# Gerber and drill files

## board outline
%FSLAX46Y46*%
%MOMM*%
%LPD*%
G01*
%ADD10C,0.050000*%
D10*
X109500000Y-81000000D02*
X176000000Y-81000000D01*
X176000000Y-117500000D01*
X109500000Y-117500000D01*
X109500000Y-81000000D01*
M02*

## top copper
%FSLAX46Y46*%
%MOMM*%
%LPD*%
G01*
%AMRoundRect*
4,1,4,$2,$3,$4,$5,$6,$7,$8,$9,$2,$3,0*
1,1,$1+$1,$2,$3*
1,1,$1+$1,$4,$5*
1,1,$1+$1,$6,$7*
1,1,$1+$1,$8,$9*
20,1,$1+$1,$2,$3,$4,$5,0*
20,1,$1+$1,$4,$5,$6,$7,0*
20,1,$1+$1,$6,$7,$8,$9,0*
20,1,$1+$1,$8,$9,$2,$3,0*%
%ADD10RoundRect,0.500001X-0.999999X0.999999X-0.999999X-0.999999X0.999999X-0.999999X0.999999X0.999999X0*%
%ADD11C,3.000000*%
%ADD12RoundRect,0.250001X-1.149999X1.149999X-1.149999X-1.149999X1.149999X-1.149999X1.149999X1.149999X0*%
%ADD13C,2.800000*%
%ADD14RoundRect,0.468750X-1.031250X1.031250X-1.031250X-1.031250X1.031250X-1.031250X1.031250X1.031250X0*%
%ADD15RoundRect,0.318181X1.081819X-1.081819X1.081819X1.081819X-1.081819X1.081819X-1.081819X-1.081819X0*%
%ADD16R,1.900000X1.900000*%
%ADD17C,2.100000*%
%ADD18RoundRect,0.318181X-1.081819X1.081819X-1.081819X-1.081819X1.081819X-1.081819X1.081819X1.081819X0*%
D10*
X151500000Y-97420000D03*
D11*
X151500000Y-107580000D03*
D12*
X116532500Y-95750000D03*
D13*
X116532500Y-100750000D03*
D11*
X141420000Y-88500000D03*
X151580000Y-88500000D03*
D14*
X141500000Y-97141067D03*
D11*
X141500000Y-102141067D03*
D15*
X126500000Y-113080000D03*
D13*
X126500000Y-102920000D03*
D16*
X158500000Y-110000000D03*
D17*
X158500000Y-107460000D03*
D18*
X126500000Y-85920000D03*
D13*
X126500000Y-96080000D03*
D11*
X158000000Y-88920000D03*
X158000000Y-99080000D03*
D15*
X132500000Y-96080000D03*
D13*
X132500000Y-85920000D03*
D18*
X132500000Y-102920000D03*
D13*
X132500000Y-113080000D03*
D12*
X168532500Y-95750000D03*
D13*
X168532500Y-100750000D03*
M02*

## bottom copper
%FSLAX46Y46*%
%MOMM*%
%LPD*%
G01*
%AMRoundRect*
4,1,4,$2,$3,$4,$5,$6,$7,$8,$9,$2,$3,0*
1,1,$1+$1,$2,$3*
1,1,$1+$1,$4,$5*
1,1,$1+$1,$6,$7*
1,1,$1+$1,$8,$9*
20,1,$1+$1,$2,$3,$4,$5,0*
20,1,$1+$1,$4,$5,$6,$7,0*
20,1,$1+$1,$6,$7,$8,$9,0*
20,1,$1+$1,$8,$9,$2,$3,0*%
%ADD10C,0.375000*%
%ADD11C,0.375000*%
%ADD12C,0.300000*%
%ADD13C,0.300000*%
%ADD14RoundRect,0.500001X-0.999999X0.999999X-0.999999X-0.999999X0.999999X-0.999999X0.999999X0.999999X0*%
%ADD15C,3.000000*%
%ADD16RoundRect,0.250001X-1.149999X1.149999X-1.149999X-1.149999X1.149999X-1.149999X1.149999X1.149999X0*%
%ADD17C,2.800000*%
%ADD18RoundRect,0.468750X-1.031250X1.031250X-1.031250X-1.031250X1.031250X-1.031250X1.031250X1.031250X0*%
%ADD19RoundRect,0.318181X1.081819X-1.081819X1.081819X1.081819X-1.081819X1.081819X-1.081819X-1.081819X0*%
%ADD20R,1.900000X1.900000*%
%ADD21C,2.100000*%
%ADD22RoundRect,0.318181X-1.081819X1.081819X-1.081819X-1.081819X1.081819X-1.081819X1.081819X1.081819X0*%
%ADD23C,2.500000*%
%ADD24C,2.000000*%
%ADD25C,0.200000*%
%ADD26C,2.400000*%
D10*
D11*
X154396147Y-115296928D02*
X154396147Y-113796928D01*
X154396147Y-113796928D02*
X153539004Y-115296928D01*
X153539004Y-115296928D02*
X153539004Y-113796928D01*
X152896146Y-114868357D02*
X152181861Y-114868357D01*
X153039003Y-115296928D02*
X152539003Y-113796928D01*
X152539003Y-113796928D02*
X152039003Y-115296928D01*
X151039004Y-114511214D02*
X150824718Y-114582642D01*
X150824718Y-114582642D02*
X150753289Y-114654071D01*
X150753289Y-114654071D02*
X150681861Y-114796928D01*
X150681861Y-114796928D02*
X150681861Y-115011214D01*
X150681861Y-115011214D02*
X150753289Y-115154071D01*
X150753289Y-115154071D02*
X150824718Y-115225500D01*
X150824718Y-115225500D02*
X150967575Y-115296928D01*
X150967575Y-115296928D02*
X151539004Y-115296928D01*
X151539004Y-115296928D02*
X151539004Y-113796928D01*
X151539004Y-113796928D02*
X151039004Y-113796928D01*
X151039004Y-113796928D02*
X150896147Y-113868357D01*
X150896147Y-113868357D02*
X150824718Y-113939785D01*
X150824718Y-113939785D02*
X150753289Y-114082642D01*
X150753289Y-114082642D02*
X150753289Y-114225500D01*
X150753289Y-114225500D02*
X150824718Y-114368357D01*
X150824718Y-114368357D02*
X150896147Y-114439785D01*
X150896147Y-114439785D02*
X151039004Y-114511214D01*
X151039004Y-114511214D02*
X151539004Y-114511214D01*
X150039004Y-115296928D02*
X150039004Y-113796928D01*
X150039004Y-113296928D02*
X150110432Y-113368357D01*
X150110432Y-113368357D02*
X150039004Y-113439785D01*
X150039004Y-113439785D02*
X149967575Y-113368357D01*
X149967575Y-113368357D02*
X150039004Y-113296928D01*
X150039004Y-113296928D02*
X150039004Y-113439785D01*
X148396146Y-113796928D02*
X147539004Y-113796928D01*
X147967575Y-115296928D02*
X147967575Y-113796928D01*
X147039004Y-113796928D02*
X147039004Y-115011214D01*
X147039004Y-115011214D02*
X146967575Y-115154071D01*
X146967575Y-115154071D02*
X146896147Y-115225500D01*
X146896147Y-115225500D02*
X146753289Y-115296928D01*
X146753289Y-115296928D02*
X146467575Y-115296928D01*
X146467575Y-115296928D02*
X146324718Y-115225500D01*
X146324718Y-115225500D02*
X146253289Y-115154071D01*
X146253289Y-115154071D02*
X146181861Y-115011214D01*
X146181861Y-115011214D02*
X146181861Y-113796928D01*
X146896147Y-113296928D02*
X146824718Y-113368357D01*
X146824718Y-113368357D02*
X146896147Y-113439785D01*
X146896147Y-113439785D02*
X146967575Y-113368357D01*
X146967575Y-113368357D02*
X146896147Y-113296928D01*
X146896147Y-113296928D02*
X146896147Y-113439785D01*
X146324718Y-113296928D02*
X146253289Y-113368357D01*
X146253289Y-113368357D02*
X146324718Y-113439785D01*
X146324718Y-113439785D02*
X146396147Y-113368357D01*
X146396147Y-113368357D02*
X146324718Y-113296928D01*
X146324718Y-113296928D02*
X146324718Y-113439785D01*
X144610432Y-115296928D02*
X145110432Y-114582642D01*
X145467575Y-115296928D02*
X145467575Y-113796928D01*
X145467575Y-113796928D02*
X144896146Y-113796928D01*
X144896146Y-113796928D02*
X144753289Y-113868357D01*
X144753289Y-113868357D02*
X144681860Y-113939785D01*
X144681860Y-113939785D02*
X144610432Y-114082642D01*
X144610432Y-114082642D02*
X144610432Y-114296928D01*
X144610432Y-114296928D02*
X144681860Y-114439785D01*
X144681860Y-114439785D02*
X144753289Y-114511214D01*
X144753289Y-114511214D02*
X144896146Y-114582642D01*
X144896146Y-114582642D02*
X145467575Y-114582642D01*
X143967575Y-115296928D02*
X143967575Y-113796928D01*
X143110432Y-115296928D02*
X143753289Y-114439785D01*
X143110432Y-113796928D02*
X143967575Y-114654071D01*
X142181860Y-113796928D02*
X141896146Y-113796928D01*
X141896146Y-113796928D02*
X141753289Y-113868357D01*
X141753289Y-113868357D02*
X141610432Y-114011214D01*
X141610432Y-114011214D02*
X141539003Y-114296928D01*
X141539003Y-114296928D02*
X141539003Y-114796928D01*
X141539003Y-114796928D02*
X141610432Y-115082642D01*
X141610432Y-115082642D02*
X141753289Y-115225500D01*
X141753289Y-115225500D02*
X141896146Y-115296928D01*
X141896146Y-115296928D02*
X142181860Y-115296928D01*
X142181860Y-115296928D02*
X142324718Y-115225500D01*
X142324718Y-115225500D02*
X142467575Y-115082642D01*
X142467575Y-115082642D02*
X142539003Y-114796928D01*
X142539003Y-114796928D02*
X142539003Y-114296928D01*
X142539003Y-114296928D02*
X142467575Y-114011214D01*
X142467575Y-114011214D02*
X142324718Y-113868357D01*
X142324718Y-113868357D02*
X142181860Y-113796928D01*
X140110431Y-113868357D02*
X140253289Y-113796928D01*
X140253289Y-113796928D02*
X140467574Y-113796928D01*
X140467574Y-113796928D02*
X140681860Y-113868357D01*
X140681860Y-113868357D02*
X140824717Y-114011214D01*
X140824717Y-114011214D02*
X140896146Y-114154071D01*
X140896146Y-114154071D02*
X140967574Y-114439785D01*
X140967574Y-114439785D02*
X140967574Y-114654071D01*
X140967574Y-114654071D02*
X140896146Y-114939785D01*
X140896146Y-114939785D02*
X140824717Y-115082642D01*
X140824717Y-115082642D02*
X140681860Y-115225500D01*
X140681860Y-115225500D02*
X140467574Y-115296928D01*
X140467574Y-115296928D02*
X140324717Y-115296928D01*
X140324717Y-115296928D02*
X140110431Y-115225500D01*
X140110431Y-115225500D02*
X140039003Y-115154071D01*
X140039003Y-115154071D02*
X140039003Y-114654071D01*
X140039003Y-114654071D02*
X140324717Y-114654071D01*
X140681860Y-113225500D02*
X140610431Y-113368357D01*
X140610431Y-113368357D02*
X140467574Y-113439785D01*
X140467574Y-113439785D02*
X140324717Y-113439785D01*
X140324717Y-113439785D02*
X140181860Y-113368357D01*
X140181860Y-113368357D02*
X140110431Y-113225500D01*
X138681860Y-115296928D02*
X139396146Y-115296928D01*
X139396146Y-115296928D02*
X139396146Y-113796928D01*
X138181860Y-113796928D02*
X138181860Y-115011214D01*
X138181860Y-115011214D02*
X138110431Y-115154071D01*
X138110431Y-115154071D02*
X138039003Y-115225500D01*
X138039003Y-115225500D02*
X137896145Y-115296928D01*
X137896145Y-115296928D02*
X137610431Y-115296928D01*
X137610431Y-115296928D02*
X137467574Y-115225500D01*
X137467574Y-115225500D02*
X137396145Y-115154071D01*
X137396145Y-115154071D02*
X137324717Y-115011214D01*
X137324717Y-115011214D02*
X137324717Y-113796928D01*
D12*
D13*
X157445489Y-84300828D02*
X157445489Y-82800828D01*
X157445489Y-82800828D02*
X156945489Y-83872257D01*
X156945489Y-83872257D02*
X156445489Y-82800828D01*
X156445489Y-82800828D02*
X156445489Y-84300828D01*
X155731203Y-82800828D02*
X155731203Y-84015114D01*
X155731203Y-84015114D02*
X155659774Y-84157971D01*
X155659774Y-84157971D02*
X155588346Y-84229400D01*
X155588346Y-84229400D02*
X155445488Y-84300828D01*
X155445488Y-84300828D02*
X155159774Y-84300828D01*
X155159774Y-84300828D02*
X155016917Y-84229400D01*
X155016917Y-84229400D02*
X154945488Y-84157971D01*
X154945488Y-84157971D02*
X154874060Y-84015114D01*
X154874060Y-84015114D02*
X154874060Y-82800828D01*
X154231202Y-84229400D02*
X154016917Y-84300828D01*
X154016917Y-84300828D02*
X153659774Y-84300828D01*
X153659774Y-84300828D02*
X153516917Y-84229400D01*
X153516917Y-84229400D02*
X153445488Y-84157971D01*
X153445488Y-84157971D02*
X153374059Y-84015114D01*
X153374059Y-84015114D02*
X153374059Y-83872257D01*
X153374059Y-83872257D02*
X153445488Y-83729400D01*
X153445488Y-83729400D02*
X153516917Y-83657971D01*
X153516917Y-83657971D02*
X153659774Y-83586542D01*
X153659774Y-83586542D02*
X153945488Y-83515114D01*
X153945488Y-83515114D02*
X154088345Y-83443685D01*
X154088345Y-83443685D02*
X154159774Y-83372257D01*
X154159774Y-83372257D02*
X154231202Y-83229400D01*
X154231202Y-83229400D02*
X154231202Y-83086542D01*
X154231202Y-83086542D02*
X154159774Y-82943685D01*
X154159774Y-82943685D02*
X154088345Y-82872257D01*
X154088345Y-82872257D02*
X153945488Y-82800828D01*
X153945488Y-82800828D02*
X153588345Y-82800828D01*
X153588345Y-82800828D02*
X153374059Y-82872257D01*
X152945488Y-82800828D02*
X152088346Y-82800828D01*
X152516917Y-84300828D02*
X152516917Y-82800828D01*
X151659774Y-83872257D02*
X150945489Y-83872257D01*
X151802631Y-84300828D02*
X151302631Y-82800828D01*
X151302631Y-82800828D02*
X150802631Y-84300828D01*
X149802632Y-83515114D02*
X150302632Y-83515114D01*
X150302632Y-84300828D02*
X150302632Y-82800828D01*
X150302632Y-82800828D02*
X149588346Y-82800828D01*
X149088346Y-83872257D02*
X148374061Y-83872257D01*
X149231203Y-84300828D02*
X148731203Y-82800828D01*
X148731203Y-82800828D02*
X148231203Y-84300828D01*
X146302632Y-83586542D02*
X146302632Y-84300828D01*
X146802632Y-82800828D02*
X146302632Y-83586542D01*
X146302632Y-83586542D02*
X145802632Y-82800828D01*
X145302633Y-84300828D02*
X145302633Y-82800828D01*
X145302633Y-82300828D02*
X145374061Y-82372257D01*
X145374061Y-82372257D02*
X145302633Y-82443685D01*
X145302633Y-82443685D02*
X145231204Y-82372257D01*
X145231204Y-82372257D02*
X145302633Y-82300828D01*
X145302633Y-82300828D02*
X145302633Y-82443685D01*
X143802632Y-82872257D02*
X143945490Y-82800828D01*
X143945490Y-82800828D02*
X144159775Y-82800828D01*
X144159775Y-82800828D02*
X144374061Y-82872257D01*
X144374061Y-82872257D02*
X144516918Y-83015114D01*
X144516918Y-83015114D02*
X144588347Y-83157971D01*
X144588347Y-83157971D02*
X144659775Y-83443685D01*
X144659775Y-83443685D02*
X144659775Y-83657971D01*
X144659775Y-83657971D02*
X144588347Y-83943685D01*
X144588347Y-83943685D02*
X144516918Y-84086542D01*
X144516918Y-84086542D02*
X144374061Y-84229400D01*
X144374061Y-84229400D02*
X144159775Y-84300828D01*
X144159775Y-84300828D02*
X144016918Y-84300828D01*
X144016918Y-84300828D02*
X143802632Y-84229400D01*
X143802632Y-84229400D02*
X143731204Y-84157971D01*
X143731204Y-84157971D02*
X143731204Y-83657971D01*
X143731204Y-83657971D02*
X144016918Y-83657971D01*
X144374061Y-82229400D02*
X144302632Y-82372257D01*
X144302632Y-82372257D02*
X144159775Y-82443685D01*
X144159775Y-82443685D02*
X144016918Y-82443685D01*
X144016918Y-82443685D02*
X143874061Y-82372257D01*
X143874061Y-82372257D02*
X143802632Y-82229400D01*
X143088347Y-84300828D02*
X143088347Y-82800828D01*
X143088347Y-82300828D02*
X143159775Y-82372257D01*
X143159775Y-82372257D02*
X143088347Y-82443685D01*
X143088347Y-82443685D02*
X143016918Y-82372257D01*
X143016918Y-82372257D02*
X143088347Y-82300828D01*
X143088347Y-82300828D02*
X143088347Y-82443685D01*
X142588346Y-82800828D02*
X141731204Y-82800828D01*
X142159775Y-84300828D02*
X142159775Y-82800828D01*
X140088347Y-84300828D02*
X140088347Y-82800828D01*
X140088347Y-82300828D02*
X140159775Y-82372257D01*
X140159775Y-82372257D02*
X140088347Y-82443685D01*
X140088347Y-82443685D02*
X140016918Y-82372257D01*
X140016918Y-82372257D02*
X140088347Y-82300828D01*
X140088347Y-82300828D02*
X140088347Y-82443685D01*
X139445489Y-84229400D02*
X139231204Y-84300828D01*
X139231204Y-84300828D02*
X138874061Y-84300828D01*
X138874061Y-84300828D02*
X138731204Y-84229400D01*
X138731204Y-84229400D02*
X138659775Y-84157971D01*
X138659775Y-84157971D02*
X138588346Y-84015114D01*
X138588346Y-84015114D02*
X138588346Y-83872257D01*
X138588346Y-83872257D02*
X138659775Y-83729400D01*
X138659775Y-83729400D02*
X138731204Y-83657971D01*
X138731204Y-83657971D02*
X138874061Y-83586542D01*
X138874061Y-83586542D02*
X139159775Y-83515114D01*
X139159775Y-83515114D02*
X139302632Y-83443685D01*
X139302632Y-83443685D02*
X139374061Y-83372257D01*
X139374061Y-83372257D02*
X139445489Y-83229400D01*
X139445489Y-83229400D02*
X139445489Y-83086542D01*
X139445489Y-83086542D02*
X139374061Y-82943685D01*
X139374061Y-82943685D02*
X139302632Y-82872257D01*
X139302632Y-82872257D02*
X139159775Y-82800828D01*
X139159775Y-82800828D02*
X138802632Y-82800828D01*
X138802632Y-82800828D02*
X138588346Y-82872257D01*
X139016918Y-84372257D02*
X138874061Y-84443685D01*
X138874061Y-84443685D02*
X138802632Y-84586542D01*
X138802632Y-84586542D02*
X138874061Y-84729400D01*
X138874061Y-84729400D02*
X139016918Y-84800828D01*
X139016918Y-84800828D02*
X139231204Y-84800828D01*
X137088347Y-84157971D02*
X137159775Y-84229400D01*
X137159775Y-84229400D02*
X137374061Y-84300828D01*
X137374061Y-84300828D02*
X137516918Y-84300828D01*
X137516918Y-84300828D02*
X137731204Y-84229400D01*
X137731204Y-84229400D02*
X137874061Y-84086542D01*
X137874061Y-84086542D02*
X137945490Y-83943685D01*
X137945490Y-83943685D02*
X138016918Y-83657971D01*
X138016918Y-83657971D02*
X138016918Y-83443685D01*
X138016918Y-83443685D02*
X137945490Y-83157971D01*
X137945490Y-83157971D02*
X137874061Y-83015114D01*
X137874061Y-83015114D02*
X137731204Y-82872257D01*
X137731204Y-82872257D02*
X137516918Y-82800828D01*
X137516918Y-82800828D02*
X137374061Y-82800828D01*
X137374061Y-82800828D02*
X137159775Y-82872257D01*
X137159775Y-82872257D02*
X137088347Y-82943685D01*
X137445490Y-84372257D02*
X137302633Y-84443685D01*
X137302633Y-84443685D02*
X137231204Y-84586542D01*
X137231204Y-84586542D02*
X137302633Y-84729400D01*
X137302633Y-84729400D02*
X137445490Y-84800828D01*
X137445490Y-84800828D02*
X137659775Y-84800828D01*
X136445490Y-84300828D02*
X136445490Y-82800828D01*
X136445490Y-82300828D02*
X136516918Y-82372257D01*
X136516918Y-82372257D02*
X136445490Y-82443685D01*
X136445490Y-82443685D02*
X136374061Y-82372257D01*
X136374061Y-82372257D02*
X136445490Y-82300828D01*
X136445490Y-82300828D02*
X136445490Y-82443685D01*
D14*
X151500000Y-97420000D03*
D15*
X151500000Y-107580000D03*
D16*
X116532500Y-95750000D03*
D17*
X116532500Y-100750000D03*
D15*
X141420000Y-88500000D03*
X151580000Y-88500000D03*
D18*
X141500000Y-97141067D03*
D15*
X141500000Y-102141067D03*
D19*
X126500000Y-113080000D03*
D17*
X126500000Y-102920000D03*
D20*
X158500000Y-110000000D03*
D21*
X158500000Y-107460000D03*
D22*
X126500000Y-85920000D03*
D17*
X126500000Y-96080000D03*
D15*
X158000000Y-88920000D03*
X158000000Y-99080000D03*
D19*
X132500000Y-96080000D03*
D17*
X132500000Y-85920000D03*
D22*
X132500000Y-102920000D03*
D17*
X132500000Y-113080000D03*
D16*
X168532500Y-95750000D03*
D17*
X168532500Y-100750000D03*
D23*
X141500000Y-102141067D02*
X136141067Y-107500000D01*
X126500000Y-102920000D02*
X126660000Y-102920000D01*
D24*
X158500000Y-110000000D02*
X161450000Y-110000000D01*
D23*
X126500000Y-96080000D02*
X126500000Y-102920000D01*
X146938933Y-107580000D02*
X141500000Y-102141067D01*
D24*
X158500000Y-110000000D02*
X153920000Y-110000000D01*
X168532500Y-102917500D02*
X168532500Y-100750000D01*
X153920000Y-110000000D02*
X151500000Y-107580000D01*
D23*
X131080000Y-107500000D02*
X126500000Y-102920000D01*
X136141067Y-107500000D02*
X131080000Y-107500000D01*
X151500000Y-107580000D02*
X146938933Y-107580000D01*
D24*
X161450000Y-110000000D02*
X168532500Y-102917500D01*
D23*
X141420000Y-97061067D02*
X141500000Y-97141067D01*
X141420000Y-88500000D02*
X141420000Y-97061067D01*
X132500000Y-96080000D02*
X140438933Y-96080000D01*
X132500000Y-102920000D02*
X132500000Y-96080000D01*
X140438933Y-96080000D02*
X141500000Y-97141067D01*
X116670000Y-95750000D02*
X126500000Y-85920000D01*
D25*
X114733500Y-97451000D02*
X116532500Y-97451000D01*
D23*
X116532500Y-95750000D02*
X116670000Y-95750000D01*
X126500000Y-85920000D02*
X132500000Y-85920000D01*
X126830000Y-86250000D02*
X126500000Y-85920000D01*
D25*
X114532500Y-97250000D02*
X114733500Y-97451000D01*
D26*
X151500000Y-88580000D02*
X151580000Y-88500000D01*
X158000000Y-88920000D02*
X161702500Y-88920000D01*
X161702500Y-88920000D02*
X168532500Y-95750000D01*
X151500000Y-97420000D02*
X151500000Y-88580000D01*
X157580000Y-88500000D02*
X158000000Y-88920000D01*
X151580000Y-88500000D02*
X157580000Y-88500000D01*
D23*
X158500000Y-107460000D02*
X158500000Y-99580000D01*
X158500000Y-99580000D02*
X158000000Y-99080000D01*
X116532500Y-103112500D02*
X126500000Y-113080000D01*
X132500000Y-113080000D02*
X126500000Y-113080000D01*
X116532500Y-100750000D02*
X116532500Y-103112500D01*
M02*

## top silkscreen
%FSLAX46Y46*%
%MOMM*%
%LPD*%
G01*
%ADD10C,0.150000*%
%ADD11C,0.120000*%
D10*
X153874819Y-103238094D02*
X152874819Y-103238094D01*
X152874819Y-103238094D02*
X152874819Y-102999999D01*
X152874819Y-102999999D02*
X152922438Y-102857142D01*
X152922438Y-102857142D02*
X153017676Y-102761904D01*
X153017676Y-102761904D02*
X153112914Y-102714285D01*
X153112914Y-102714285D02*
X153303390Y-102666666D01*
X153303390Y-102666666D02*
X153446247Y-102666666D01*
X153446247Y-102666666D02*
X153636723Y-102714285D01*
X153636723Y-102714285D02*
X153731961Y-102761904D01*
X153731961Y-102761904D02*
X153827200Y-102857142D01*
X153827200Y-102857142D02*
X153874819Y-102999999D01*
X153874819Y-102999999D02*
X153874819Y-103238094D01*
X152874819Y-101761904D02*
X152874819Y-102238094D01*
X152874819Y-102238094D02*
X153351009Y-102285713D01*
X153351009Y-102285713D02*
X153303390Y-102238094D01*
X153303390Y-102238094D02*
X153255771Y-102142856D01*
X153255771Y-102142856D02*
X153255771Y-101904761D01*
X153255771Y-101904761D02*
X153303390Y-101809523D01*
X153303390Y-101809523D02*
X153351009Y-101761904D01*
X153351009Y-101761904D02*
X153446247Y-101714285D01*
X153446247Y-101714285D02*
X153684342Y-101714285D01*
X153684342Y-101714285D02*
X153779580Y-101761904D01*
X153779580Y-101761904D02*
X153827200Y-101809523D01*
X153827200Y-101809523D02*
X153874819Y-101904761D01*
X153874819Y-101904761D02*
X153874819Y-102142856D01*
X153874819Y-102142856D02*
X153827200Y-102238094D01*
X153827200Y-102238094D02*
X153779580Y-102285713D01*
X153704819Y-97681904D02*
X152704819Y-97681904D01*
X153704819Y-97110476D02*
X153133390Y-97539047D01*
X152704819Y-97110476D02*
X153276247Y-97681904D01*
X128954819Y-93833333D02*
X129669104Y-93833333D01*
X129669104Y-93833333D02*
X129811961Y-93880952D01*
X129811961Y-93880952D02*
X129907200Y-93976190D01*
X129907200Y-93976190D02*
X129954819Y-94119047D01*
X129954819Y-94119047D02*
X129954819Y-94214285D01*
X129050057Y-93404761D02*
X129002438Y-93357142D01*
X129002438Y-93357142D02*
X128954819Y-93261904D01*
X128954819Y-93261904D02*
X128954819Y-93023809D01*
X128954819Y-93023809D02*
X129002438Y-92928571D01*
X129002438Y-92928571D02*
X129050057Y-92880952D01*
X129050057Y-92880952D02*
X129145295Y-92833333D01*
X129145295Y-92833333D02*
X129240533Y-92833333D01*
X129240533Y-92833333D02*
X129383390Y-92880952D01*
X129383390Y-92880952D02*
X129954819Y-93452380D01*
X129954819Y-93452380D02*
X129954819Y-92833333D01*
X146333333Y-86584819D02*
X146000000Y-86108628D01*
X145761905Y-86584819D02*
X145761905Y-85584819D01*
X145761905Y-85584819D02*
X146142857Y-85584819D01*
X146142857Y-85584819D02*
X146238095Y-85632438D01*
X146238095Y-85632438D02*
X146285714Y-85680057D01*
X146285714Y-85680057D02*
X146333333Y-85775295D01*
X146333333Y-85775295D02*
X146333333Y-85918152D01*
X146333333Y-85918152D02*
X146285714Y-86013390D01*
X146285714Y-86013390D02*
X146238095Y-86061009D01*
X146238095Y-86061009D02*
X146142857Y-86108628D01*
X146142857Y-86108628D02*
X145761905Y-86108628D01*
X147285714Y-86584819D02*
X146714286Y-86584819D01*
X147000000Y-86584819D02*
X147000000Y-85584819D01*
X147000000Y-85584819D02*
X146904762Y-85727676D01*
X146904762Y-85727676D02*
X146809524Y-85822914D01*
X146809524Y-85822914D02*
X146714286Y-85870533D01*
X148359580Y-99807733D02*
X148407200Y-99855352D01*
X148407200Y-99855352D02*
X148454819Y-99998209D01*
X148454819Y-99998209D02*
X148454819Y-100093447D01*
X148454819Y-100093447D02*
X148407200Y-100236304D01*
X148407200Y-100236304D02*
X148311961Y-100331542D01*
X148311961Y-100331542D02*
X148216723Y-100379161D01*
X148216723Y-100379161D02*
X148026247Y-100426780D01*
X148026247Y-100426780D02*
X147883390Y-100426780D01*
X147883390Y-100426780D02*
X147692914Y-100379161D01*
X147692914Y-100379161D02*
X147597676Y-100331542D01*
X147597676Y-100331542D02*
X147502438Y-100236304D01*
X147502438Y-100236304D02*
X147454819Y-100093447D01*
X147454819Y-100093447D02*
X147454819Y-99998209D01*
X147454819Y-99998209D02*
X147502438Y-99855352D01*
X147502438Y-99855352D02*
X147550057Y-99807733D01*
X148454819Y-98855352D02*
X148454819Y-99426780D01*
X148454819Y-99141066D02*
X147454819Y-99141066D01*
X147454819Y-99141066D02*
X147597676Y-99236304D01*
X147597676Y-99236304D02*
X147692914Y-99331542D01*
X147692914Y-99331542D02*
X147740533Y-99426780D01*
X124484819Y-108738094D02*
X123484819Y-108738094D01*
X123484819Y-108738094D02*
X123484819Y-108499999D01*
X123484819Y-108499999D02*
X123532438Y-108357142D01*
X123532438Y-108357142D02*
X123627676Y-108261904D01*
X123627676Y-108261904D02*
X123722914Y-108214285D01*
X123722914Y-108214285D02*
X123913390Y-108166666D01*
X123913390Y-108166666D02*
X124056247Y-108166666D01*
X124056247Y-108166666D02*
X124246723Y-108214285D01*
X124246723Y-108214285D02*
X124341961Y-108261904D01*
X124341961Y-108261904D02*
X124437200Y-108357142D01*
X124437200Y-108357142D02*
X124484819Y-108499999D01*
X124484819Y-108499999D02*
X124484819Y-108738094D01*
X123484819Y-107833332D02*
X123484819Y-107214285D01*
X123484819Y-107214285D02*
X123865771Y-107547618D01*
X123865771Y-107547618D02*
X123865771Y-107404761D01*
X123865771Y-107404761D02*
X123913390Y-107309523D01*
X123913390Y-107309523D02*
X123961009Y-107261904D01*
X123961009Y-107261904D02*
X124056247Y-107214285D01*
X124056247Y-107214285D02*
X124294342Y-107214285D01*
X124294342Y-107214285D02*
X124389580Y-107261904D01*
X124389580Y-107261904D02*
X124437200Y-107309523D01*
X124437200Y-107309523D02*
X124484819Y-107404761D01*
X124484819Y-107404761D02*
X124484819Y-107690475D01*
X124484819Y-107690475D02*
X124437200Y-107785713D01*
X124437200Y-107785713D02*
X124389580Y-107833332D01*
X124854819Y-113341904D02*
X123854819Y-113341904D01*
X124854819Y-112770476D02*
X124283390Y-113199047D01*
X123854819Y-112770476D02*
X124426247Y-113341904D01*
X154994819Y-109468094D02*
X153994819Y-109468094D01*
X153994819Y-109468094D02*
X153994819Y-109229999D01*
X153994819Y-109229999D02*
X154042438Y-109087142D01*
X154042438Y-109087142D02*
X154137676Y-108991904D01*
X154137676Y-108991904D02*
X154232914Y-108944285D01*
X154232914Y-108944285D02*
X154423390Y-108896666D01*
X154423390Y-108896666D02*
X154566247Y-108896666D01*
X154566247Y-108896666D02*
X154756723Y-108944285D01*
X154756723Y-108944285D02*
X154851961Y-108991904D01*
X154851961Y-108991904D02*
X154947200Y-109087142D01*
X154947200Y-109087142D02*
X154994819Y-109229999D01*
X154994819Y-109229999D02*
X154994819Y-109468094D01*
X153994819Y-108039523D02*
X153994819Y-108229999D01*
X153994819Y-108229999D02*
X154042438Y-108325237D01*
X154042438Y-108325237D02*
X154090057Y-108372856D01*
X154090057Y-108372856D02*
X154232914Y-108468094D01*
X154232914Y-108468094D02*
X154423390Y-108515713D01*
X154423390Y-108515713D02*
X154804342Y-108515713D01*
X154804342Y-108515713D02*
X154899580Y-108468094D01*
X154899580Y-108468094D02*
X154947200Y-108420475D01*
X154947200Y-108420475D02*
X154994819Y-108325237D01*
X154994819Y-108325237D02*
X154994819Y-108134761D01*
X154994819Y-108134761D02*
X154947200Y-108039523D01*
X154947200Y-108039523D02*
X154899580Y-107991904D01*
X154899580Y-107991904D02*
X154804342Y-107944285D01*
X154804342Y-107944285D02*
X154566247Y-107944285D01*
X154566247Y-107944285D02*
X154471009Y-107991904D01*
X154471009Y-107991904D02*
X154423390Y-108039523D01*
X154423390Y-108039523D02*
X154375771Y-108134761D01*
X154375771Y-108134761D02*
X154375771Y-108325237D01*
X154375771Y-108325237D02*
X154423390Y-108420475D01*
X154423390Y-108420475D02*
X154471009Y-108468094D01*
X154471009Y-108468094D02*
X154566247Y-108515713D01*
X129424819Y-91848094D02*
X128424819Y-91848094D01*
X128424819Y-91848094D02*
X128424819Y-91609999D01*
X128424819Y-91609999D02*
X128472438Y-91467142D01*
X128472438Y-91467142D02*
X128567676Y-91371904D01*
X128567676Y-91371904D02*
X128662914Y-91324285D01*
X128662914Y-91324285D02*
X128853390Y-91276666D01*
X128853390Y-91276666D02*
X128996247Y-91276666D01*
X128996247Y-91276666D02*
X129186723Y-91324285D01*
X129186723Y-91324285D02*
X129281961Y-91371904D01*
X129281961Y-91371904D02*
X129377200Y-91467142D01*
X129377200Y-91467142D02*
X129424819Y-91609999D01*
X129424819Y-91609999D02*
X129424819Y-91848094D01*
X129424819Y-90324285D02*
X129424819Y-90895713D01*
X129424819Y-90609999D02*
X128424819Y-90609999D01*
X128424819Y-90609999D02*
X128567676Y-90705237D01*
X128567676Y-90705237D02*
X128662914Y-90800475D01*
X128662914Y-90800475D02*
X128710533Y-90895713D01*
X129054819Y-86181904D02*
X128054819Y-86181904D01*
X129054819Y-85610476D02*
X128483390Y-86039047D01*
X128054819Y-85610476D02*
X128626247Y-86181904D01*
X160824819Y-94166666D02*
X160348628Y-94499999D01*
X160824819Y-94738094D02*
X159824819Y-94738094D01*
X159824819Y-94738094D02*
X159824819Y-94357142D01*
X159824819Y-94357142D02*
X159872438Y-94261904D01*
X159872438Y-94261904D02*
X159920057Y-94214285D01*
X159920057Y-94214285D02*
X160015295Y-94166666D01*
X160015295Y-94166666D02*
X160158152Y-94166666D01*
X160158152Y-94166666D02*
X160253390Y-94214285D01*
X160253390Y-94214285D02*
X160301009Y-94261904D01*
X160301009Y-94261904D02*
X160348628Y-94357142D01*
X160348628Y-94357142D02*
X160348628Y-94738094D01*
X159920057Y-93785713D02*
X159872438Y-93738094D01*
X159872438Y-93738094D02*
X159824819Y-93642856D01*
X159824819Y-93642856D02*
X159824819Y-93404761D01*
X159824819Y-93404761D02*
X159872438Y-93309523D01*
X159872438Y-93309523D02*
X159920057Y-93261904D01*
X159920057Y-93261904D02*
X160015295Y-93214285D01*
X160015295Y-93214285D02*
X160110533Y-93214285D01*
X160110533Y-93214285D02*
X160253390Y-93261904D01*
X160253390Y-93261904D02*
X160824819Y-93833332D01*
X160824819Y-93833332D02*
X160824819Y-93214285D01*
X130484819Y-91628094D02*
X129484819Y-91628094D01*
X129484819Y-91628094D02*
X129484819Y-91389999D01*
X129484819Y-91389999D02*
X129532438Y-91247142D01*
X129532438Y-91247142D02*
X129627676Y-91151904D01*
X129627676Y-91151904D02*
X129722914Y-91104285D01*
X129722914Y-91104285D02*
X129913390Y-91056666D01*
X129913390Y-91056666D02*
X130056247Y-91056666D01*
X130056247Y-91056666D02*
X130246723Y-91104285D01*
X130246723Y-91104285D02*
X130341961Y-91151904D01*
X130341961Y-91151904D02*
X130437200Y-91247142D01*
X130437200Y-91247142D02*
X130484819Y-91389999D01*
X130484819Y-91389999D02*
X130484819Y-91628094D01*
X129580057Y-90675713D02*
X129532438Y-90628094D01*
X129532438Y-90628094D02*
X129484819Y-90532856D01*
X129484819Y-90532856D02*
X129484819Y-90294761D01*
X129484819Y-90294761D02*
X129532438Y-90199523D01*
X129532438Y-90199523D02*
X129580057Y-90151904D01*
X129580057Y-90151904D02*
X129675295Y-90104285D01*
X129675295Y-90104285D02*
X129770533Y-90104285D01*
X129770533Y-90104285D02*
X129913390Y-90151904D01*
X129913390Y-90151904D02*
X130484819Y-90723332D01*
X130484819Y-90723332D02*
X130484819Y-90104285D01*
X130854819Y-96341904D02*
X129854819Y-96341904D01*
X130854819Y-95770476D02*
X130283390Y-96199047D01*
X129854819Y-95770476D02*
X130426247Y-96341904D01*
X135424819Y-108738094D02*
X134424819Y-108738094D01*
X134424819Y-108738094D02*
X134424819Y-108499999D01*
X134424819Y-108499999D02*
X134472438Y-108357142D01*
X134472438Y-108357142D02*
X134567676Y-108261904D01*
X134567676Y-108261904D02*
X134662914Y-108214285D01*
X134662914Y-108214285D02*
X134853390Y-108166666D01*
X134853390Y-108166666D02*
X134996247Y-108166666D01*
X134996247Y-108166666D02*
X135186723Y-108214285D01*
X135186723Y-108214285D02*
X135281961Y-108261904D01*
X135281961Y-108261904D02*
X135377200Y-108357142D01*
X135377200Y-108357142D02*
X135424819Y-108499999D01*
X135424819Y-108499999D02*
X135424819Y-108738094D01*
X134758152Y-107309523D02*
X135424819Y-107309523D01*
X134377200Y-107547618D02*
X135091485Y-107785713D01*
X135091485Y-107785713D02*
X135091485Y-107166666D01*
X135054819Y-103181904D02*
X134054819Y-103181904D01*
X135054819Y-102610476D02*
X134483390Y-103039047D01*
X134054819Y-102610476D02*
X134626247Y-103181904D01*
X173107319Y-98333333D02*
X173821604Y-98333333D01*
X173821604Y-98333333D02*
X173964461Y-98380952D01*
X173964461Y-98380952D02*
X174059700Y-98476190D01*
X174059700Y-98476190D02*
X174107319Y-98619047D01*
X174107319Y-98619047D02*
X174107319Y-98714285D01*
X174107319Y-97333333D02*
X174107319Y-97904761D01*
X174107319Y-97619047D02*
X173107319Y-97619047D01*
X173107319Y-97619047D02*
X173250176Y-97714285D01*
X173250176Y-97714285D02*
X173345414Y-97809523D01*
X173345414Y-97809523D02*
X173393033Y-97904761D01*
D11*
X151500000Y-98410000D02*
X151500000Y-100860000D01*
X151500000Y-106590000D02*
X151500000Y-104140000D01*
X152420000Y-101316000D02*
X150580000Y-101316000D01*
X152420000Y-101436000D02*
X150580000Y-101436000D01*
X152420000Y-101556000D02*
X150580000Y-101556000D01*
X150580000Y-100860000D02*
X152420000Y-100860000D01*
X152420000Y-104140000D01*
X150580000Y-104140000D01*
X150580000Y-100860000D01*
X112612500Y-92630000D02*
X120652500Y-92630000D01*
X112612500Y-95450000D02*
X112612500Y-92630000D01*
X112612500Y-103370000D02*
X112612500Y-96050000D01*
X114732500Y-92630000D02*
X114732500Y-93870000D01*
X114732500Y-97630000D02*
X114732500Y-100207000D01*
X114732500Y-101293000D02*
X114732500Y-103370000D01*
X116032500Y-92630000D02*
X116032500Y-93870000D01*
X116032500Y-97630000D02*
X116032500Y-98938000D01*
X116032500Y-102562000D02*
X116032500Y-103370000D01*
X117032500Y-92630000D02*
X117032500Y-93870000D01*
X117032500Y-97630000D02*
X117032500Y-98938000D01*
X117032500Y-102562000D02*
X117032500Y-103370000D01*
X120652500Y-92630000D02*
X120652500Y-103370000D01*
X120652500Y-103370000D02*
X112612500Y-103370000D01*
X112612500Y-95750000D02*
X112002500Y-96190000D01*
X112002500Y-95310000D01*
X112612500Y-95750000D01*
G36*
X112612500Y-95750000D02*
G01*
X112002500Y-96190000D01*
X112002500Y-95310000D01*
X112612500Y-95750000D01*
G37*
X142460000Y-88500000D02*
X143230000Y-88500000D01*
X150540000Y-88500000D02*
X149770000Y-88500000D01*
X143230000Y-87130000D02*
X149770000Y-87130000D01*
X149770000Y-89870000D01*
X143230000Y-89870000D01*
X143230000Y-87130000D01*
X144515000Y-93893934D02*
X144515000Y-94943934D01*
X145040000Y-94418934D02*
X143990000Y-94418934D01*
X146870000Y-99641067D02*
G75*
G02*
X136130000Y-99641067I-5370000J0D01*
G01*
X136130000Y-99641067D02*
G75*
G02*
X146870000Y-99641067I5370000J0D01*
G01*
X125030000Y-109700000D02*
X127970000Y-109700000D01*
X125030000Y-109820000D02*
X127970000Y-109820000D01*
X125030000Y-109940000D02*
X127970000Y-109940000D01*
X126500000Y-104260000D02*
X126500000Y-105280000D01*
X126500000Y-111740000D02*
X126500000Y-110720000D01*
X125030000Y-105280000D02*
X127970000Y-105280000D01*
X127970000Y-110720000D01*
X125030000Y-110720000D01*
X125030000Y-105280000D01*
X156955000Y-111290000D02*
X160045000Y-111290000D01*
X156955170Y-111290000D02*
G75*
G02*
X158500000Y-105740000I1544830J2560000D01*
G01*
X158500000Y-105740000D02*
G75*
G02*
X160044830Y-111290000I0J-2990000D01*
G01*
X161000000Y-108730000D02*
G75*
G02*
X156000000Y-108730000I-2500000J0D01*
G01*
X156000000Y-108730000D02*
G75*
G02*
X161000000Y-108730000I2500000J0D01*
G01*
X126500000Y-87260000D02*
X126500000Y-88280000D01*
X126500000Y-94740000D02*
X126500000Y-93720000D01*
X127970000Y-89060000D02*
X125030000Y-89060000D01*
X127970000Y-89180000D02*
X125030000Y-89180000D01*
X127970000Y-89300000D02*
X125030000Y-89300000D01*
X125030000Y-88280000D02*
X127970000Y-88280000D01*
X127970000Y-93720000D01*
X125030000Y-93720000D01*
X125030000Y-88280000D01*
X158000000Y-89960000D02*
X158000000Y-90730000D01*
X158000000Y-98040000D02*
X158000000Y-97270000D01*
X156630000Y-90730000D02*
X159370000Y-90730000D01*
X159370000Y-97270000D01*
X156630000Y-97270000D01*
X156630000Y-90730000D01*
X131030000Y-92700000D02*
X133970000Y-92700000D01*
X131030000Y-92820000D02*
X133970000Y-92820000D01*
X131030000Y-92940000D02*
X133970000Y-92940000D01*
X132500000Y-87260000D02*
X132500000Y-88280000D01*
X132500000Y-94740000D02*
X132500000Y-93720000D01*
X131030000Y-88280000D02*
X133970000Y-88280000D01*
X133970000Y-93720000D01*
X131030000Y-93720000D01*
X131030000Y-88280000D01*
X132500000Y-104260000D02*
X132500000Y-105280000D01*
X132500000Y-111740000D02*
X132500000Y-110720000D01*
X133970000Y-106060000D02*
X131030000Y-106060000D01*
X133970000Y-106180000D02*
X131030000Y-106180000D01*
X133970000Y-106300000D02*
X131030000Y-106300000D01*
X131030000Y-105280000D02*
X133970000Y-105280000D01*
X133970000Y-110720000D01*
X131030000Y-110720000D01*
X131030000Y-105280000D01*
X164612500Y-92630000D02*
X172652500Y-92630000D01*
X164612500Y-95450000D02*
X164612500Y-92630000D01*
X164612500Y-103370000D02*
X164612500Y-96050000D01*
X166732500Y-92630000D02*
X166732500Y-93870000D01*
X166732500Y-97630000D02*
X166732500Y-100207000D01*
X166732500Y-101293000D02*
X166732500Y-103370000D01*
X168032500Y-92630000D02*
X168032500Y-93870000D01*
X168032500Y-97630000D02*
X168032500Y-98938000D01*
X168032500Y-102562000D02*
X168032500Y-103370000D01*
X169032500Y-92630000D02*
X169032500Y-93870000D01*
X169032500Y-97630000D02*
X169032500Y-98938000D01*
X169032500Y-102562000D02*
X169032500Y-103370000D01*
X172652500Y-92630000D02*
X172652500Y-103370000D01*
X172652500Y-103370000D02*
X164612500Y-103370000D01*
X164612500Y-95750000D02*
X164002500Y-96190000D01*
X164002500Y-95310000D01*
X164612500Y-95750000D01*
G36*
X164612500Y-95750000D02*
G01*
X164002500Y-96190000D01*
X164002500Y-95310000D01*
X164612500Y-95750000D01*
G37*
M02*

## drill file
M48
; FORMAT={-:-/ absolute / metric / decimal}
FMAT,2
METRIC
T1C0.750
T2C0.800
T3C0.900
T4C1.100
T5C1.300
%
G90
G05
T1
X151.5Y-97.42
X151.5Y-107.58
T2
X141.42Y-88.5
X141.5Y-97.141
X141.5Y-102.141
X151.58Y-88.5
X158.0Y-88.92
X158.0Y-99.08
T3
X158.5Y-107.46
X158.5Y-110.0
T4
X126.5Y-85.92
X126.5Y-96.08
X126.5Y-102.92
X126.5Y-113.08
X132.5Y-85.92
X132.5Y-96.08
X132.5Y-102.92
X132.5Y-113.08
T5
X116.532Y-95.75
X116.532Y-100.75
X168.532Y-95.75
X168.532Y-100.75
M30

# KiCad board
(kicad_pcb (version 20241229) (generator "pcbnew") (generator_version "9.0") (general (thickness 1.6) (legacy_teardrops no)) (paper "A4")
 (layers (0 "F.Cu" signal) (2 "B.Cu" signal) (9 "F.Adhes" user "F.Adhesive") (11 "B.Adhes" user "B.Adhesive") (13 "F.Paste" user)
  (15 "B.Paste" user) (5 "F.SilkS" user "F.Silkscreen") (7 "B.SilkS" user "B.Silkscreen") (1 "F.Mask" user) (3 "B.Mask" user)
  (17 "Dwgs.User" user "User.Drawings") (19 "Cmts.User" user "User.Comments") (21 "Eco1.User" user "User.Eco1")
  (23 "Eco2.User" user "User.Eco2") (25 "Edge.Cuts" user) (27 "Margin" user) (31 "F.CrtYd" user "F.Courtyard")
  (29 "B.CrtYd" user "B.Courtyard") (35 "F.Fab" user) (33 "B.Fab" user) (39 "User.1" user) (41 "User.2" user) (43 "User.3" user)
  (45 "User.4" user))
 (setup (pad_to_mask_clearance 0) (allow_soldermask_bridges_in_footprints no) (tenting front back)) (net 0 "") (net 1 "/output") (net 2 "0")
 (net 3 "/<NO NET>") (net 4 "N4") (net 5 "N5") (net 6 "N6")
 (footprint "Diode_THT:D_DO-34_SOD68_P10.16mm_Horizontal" (layer "F.Cu") (at 151.5 97.42 -90)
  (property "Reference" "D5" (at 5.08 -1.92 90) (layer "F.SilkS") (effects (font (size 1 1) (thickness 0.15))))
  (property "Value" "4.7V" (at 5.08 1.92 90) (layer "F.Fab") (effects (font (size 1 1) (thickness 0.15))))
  (fp_line (start 0.99 0) (end 3.44 0) (stroke (width 0.12) (type solid)) (layer "F.SilkS"))
  (fp_line (start 9.17 0) (end 6.72 0) (stroke (width 0.12) (type solid)) (layer "F.SilkS"))
  (fp_line (start 3.896 -0.92) (end 3.896 0.92) (stroke (width 0.12) (type solid)) (layer "F.SilkS"))
  (fp_line (start 4.016 -0.92) (end 4.016 0.92) (stroke (width 0.12) (type solid)) (layer "F.SilkS"))
  (fp_line (start 4.136 -0.92) (end 4.136 0.92) (stroke (width 0.12) (type solid)) (layer "F.SilkS"))
  (fp_rect (start 3.44 -0.92) (end 6.72 0.92) (stroke (width 0.12) (type solid)) (fill no) (layer "F.SilkS"))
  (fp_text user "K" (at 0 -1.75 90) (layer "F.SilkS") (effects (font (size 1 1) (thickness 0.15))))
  (pad "1" thru_hole roundrect (at 0 0 270) (size 3 3) (drill 0.75) (layers "*.Cu" "*.Mask") (remove_unused_layers no)
   (roundrect_rratio 0.166667) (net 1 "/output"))
  (pad "2" thru_hole circle (at 10.16 0 270) (size 3 3) (drill 0.75) (layers "*.Cu" "*.Mask") (remove_unused_layers no) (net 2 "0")))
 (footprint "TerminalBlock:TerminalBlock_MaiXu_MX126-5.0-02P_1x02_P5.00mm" (layer "F.Cu") (at 116.5325 95.75 -90)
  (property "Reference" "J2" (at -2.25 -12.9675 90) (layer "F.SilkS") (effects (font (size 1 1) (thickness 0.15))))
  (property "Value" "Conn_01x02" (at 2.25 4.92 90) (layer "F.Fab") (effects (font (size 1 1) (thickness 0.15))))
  (fp_line (start -3.12 3.92) (end -3.12 -4.12) (stroke (width 0.12) (type solid)) (layer "F.SilkS"))
  (fp_line (start -0.3 3.92) (end -3.12 3.92) (stroke (width 0.12) (type solid)) (layer "F.SilkS"))
  (fp_line (start 7.62 3.92) (end 0.3 3.92) (stroke (width 0.12) (type solid)) (layer "F.SilkS"))
  (fp_line (start -3.12 1.8) (end -1.88 1.8) (stroke (width 0.12) (type solid)) (layer "F.SilkS"))
  (fp_line (start 1.88 1.8) (end 4.457 1.8) (stroke (width 0.12) (type solid)) (layer "F.SilkS"))
  (fp_line (start 5.543 1.8) (end 7.62 1.8) (stroke (width 0.12) (type solid)) (layer "F.SilkS"))
  (fp_line (start -3.12 0.5) (end -1.88 0.5) (stroke (width 0.12) (type solid)) (layer "F.SilkS"))
  (fp_line (start 1.88 0.5) (end 3.188 0.5) (stroke (width 0.12) (type solid)) (layer "F.SilkS"))
  (fp_line (start 6.812 0.5) (end 7.62 0.5) (stroke (width 0.12) (type solid)) (layer "F.SilkS"))
  (fp_line (start -3.12 -0.5) (end -1.88 -0.5) (stroke (width 0.12) (type solid)) (layer "F.SilkS"))
  (fp_line (start 1.88 -0.5) (end 3.188 -0.5) (stroke (width 0.12) (type solid)) (layer "F.SilkS"))
  (fp_line (start 6.812 -0.5) (end 7.62 -0.5) (stroke (width 0.12) (type solid)) (layer "F.SilkS"))
  (fp_line (start -3.12 -4.12) (end 7.62 -4.12) (stroke (width 0.12) (type solid)) (layer "F.SilkS"))
  (fp_line (start 7.62 -4.12) (end 7.62 3.92) (stroke (width 0.12) (type solid)) (layer "F.SilkS"))
  (fp_poly (pts (xy 0 3.92) (xy 0.44 4.53) (xy -0.44 4.53)) (stroke (width 0.12) (type solid)) (fill yes) (layer "F.SilkS"))
  (pad "1" thru_hole roundrect (at 0 0 270) (size 2.8 2.8) (drill 1.3) (layers "*.Cu" "*.Mask") (remove_unused_layers no)
   (roundrect_rratio 0.089286) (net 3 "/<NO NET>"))
  (pad "2" thru_hole circle (at 5 0 270) (size 2.8 2.8) (drill 1.3) (layers "*.Cu" "*.Mask") (remove_unused_layers no) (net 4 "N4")))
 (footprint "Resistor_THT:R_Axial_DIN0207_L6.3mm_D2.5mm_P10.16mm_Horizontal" (layer "F.Cu") (at 141.42 88.5)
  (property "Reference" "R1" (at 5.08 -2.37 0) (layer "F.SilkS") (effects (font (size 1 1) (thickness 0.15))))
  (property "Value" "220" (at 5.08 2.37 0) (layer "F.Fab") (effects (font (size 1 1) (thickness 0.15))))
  (fp_line (start 1.04 0) (end 1.81 0) (stroke (width 0.12) (type solid)) (layer "F.SilkS"))
  (fp_line (start 9.12 0) (end 8.35 0) (stroke (width 0.12) (type solid)) (layer "F.SilkS"))
  (fp_rect (start 1.81 -1.37) (end 8.35 1.37) (stroke (width 0.12) (type solid)) (fill no) (layer "F.SilkS"))
  (pad "1" thru_hole circle (at 0 0) (size 3 3) (drill 0.8) (layers "*.Cu" "*.Mask") (remove_unused_layers no) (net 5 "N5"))
  (pad "2" thru_hole circle (at 10.16 0) (size 3 3) (drill 0.8) (layers "*.Cu" "*.Mask") (remove_unused_layers no) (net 1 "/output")))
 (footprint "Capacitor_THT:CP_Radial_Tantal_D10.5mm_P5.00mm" (layer "F.Cu") (at 141.5 97.141067 -90)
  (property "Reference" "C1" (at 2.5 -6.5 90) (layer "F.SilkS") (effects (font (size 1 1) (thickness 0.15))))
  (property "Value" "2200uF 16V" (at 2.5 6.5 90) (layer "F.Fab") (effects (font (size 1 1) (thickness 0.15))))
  (fp_line (start -3.247133 -3.015) (end -2.197133 -3.015) (stroke (width 0.12) (type solid)) (layer "F.SilkS"))
  (fp_line (start -2.722133 -3.54) (end -2.722133 -2.49) (stroke (width 0.12) (type solid)) (layer "F.SilkS"))
  (fp_circle (center 2.5 0) (end 7.87 0) (stroke (width 0.12) (type solid)) (fill no) (layer "F.SilkS"))
  (pad "1" thru_hole roundrect (at 0 0 270) (size 3 3) (drill 0.8) (layers "*.Cu" "*.Mask") (remove_unused_layers no)
   (roundrect_rratio 0.15625) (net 5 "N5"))
  (pad "2" thru_hole circle (at 5 0 270) (size 3 3) (drill 0.8) (layers "*.Cu" "*.Mask") (remove_unused_layers no) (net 2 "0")))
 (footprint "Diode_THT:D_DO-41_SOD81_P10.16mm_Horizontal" (layer "F.Cu") (at 126.5 113.08 90)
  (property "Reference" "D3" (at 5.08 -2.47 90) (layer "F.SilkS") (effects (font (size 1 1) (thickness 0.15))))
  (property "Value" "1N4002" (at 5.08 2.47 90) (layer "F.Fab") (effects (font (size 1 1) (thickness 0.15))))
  (fp_line (start 3.38 -1.47) (end 3.38 1.47) (stroke (width 0.12) (type solid)) (layer "F.SilkS"))
  (fp_line (start 3.26 -1.47) (end 3.26 1.47) (stroke (width 0.12) (type solid)) (layer "F.SilkS"))
  (fp_line (start 3.14 -1.47) (end 3.14 1.47) (stroke (width 0.12) (type solid)) (layer "F.SilkS"))
  (fp_line (start 8.82 0) (end 7.8 0) (stroke (width 0.12) (type solid)) (layer "F.SilkS"))
  (fp_line (start 1.34 0) (end 2.36 0) (stroke (width 0.12) (type solid)) (layer "F.SilkS"))
  (fp_rect (start 2.36 -1.47) (end 7.8 1.47) (stroke (width 0.12) (type solid)) (fill no) (layer "F.SilkS"))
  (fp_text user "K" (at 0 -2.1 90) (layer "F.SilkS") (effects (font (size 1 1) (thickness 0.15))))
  (pad "1" thru_hole roundrect (at 0 0 90) (size 2.8 2.8) (drill 1.1) (layers "*.Cu" "*.Mask") (remove_unused_layers no)
   (roundrect_rratio 0.113636) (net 4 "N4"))
  (pad "2" thru_hole circle (at 10.16 0 90) (size 2.8 2.8) (drill 1.1) (layers "*.Cu" "*.Mask") (remove_unused_layers no) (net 2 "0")))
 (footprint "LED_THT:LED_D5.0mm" (layer "F.Cu") (at 158.5 110 90)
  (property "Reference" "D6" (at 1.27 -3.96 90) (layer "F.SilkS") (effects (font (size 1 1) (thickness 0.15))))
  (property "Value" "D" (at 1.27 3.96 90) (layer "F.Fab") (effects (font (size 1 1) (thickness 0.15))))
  (fp_line (start -1.29 -1.545) (end -1.29 1.545) (stroke (width 0.12) (type solid)) (layer "F.SilkS"))
  (fp_arc (start -1.29 -1.54483) (mid 2.071779 -2.880495) (end 4.26 0) (stroke (width 0.12) (type solid)) (layer "F.SilkS"))
  (fp_arc (start 4.26 0) (mid 2.071779 2.880495) (end -1.29 1.54483) (stroke (width 0.12) (type solid)) (layer "F.SilkS"))
  (fp_circle (center 1.27 0) (end 3.77 0) (stroke (width 0.12) (type solid)) (fill no) (layer "F.SilkS"))
  (pad "1" thru_hole rect (at 0 0 90) (size 1.9 1.9) (drill 0.9) (layers "*.Cu" "*.Mask") (remove_unused_layers no) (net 2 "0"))
  (pad "2" thru_hole circle (at 2.54 0 90) (size 2.1 2.1) (drill 0.9) (layers "*.Cu" "*.Mask") (remove_unused_layers no) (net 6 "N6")))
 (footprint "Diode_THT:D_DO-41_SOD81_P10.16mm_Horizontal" (layer "F.Cu") (at 126.5 85.92 -90)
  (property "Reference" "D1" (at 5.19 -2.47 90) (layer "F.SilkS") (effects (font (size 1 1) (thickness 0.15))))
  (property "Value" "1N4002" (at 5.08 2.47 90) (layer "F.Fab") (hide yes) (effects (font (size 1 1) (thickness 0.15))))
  (fp_line (start 1.34 0) (end 2.36 0) (stroke (width 0.12) (type solid)) (layer "F.SilkS"))
  (fp_line (start 8.82 0) (end 7.8 0) (stroke (width 0.12) (type solid)) (layer "F.SilkS"))
  (fp_line (start 3.14 -1.47) (end 3.14 1.47) (stroke (width 0.12) (type solid)) (layer "F.SilkS"))
  (fp_line (start 3.26 -1.47) (end 3.26 1.47) (stroke (width 0.12) (type solid)) (layer "F.SilkS"))
  (fp_line (start 3.38 -1.47) (end 3.38 1.47) (stroke (width 0.12) (type solid)) (layer "F.SilkS"))
  (fp_rect (start 2.36 -1.47) (end 7.8 1.47) (stroke (width 0.12) (type solid)) (fill no) (layer "F.SilkS"))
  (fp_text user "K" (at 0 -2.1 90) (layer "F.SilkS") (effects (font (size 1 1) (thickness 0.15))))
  (pad "1" thru_hole roundrect (at 0 0 270) (size 2.8 2.8) (drill 1.1) (layers "*.Cu" "*.Mask") (remove_unused_layers no)
   (roundrect_rratio 0.113636) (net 3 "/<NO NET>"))
  (pad "2" thru_hole circle (at 10.16 0 270) (size 2.8 2.8) (drill 1.1) (layers "*.Cu" "*.Mask") (remove_unused_layers no) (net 2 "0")))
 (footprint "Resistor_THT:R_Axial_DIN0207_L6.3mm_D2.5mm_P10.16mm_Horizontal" (layer "F.Cu") (at 158 88.92 -90)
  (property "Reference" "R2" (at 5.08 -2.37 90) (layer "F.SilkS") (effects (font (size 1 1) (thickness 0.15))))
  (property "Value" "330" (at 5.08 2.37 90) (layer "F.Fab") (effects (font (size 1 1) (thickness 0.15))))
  (fp_line (start 1.04 0) (end 1.81 0) (stroke (width 0.12) (type solid)) (layer "F.SilkS"))
  (fp_line (start 9.12 0) (end 8.35 0) (stroke (width 0.12) (type solid)) (layer "F.SilkS"))
  (fp_rect (start 1.81 -1.37) (end 8.35 1.37) (stroke (width 0.12) (type solid)) (fill no) (layer "F.SilkS"))
  (pad "1" thru_hole circle (at 0 0 270) (size 3 3) (drill 0.8) (layers "*.Cu" "*.Mask") (remove_unused_layers no) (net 1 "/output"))
  (pad "2" thru_hole circle (at 10.16 0 270) (size 3 3) (drill 0.8) (layers "*.Cu" "*.Mask") (remove_unused_layers no) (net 6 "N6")))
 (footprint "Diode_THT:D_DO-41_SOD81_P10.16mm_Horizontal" (layer "F.Cu") (at 132.5 96.08 90)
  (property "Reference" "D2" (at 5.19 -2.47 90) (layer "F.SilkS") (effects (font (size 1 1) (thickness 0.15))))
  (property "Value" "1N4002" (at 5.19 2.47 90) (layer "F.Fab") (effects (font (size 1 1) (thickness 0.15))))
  (fp_line (start 3.38 -1.47) (end 3.38 1.47) (stroke (width 0.12) (type solid)) (layer "F.SilkS"))
  (fp_line (start 3.26 -1.47) (end 3.26 1.47) (stroke (width 0.12) (type solid)) (layer "F.SilkS"))
  (fp_line (start 3.14 -1.47) (end 3.14 1.47) (stroke (width 0.12) (type solid)) (layer "F.SilkS"))
  (fp_line (start 8.82 0) (end 7.8 0) (stroke (width 0.12) (type solid)) (layer "F.SilkS"))
  (fp_line (start 1.34 0) (end 2.36 0) (stroke (width 0.12) (type solid)) (layer "F.SilkS"))
  (fp_rect (start 2.36 -1.47) (end 7.8 1.47) (stroke (width 0.12) (type solid)) (fill no) (layer "F.SilkS"))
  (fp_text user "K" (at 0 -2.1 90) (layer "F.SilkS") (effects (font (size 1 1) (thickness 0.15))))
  (pad "1" thru_hole roundrect (at 0 0 90) (size 2.8 2.8) (drill 1.1) (layers "*.Cu" "*.Mask") (remove_unused_layers no)
   (roundrect_rratio 0.113636) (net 5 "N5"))
  (pad "2" thru_hole circle (at 10.16 0 90) (size 2.8 2.8) (drill 1.1) (layers "*.Cu" "*.Mask") (remove_unused_layers no)
   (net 3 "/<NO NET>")))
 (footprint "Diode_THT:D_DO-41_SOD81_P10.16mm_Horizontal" (layer "F.Cu") (at 132.5 102.92 -90)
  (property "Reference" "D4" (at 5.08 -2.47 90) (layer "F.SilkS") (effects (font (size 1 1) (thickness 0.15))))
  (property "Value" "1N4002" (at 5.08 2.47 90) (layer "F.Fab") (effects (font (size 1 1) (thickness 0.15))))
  (fp_line (start 1.34 0) (end 2.36 0) (stroke (width 0.12) (type solid)) (layer "F.SilkS"))
  (fp_line (start 8.82 0) (end 7.8 0) (stroke (width 0.12) (type solid)) (layer "F.SilkS"))
  (fp_line (start 3.14 -1.47) (end 3.14 1.47) (stroke (width 0.12) (type solid)) (layer "F.SilkS"))
  (fp_line (start 3.26 -1.47) (end 3.26 1.47) (stroke (width 0.12) (type solid)) (layer "F.SilkS"))
  (fp_line (start 3.38 -1.47) (end 3.38 1.47) (stroke (width 0.12) (type solid)) (layer "F.SilkS"))
  (fp_rect (start 2.36 -1.47) (end 7.8 1.47) (stroke (width 0.12) (type solid)) (fill no) (layer "F.SilkS"))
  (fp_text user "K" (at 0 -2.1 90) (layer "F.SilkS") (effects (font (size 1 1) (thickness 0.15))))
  (pad "1" thru_hole roundrect (at 0 0 270) (size 2.8 2.8) (drill 1.1) (layers "*.Cu" "*.Mask") (remove_unused_layers no)
   (roundrect_rratio 0.113636) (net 5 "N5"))
  (pad "2" thru_hole circle (at 10.16 0 270) (size 2.8 2.8) (drill 1.1) (layers "*.Cu" "*.Mask") (remove_unused_layers no) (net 4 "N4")))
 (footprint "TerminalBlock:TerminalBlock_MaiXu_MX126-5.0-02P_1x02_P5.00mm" (layer "F.Cu") (at 168.5325 95.75 -90)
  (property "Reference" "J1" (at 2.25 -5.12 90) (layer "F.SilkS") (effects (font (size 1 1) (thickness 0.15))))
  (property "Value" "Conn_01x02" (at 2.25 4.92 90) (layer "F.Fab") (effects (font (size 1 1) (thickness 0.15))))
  (fp_line (start -3.12 3.92) (end -3.12 -4.12) (stroke (width 0.12) (type solid)) (layer "F.SilkS"))
  (fp_line (start -0.3 3.92) (end -3.12 3.92) (stroke (width 0.12) (type solid)) (layer "F.SilkS"))
  (fp_line (start 7.62 3.92) (end 0.3 3.92) (stroke (width 0.12) (type solid)) (layer "F.SilkS"))
  (fp_line (start -3.12 1.8) (end -1.88 1.8) (stroke (width 0.12) (type solid)) (layer "F.SilkS"))
  (fp_line (start 1.88 1.8) (end 4.457 1.8) (stroke (width 0.12) (type solid)) (layer "F.SilkS"))
  (fp_line (start 5.543 1.8) (end 7.62 1.8) (stroke (width 0.12) (type solid)) (layer "F.SilkS"))
  (fp_line (start -3.12 0.5) (end -1.88 0.5) (stroke (width 0.12) (type solid)) (layer "F.SilkS"))
  (fp_line (start 1.88 0.5) (end 3.188 0.5) (stroke (width 0.12) (type solid)) (layer "F.SilkS"))
  (fp_line (start 6.812 0.5) (end 7.62 0.5) (stroke (width 0.12) (type solid)) (layer "F.SilkS"))
  (fp_line (start -3.12 -0.5) (end -1.88 -0.5) (stroke (width 0.12) (type solid)) (layer "F.SilkS"))
  (fp_line (start 1.88 -0.5) (end 3.188 -0.5) (stroke (width 0.12) (type solid)) (layer "F.SilkS"))
  (fp_line (start 6.812 -0.5) (end 7.62 -0.5) (stroke (width 0.12) (type solid)) (layer "F.SilkS"))
  (fp_line (start -3.12 -4.12) (end 7.62 -4.12) (stroke (width 0.12) (type solid)) (layer "F.SilkS"))
  (fp_line (start 7.62 -4.12) (end 7.62 3.92) (stroke (width 0.12) (type solid)) (layer "F.SilkS"))
  (fp_poly (pts (xy 0 3.92) (xy 0.44 4.53) (xy -0.44 4.53)) (stroke (width 0.12) (type solid)) (fill yes) (layer "F.SilkS"))
  (pad "1" thru_hole roundrect (at 0 0 270) (size 2.8 2.8) (drill 1.3) (layers "*.Cu" "*.Mask") (remove_unused_layers no)
   (roundrect_rratio 0.089286) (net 1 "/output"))
  (pad "2" thru_hole circle (at 5 0 270) (size 2.8 2.8) (drill 1.3) (layers "*.Cu" "*.Mask") (remove_unused_layers no) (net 2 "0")))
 (gr_rect (start 109.5 81) (end 176 117.5) (stroke (width 0.05) (type default)) (fill no) (layer "Edge.Cuts"))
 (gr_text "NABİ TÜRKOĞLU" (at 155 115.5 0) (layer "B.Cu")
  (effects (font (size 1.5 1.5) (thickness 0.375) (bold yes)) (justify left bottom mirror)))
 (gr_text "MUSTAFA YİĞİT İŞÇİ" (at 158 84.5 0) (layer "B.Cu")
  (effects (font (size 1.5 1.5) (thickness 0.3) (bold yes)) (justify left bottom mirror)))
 (segment (start 141.5 102.141067) (end 136.141067 107.5) (width 2.5) (layer "B.Cu") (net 2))
 (segment (start 126.5 102.92) (end 126.66 102.92) (width 2.5) (layer "B.Cu") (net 2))
 (segment (start 158.5 110) (end 161.45 110) (width 2) (layer "B.Cu") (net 2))
 (segment (start 126.5 96.08) (end 126.5 102.92) (width 2.5) (layer "B.Cu") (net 2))
 (segment (start 146.938933 107.58) (end 141.5 102.141067) (width 2.5) (layer "B.Cu") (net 2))
 (segment (start 158.5 110) (end 153.92 110) (width 2) (layer "B.Cu") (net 2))
 (segment (start 168.5325 102.9175) (end 168.5325 100.75) (width 2) (layer "B.Cu") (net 2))
 (segment (start 153.92 110) (end 151.5 107.58) (width 2) (layer "B.Cu") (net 2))
 (segment (start 131.08 107.5) (end 126.5 102.92) (width 2.5) (layer "B.Cu") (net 2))
 (segment (start 136.141067 107.5) (end 131.08 107.5) (width 2.5) (layer "B.Cu") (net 2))
 (segment (start 151.5 107.58) (end 146.938933 107.58) (width 2.5) (layer "B.Cu") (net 2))
 (segment (start 161.45 110) (end 168.5325 102.9175) (width 2) (layer "B.Cu") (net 2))
 (segment (start 141.42 97.061067) (end 141.5 97.141067) (width 2.5) (layer "B.Cu") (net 5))
 (segment (start 141.42 88.5) (end 141.42 97.061067) (width 2.5) (layer "B.Cu") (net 5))
 (segment (start 132.5 96.08) (end 140.438933 96.08) (width 2.5) (layer "B.Cu") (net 5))
 (segment (start 132.5 102.92) (end 132.5 96.08) (width 2.5) (layer "B.Cu") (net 5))
 (segment (start 140.438933 96.08) (end 141.5 97.141067) (width 2.5) (layer "B.Cu") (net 5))
 (segment (start 116.67 95.75) (end 126.5 85.92) (width 2.5) (layer "B.Cu") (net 3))
 (segment (start 114.7335 97.451) (end 116.5325 97.451) (width 0.2) (layer "B.Cu") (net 3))
 (segment (start 116.5325 95.75) (end 116.67 95.75) (width 2.5) (layer "B.Cu") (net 3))
 (segment (start 126.5 85.92) (end 132.5 85.92) (width 2.5) (layer "B.Cu") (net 3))
 (segment (start 126.83 86.25) (end 126.5 85.92) (width 2.5) (layer "B.Cu") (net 3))
 (segment (start 114.5325 97.25) (end 114.7335 97.451) (width 0.2) (layer "B.Cu") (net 3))
 (segment (start 151.5 88.58) (end 151.58 88.5) (width 2.4) (layer "B.Cu") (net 1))
 (segment (start 158 88.92) (end 161.7025 88.92) (width 2.4) (layer "B.Cu") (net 1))
 (segment (start 161.7025 88.92) (end 168.5325 95.75) (width 2.4) (layer "B.Cu") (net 1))
 (segment (start 151.5 97.42) (end 151.5 88.58) (width 2.4) (layer "B.Cu") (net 1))
 (segment (start 157.58 88.5) (end 158 88.92) (width 2.4) (layer "B.Cu") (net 1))
 (segment (start 151.58 88.5) (end 157.58 88.5) (width 2.4) (layer "B.Cu") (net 1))
 (segment (start 158.5 107.46) (end 158.5 99.58) (width 2.5) (layer "B.Cu") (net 6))
 (segment (start 158.5 99.58) (end 158 99.08) (width 2.5) (layer "B.Cu") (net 6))
 (segment (start 116.5325 103.1125) (end 126.5 113.08) (width 2.5) (layer "B.Cu") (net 4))
 (segment (start 132.5 113.08) (end 126.5 113.08) (width 2.5) (layer "B.Cu") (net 4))
 (segment (start 116.5325 100.75) (end 116.5325 103.1125) (width 2.5) (layer "B.Cu") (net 4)))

